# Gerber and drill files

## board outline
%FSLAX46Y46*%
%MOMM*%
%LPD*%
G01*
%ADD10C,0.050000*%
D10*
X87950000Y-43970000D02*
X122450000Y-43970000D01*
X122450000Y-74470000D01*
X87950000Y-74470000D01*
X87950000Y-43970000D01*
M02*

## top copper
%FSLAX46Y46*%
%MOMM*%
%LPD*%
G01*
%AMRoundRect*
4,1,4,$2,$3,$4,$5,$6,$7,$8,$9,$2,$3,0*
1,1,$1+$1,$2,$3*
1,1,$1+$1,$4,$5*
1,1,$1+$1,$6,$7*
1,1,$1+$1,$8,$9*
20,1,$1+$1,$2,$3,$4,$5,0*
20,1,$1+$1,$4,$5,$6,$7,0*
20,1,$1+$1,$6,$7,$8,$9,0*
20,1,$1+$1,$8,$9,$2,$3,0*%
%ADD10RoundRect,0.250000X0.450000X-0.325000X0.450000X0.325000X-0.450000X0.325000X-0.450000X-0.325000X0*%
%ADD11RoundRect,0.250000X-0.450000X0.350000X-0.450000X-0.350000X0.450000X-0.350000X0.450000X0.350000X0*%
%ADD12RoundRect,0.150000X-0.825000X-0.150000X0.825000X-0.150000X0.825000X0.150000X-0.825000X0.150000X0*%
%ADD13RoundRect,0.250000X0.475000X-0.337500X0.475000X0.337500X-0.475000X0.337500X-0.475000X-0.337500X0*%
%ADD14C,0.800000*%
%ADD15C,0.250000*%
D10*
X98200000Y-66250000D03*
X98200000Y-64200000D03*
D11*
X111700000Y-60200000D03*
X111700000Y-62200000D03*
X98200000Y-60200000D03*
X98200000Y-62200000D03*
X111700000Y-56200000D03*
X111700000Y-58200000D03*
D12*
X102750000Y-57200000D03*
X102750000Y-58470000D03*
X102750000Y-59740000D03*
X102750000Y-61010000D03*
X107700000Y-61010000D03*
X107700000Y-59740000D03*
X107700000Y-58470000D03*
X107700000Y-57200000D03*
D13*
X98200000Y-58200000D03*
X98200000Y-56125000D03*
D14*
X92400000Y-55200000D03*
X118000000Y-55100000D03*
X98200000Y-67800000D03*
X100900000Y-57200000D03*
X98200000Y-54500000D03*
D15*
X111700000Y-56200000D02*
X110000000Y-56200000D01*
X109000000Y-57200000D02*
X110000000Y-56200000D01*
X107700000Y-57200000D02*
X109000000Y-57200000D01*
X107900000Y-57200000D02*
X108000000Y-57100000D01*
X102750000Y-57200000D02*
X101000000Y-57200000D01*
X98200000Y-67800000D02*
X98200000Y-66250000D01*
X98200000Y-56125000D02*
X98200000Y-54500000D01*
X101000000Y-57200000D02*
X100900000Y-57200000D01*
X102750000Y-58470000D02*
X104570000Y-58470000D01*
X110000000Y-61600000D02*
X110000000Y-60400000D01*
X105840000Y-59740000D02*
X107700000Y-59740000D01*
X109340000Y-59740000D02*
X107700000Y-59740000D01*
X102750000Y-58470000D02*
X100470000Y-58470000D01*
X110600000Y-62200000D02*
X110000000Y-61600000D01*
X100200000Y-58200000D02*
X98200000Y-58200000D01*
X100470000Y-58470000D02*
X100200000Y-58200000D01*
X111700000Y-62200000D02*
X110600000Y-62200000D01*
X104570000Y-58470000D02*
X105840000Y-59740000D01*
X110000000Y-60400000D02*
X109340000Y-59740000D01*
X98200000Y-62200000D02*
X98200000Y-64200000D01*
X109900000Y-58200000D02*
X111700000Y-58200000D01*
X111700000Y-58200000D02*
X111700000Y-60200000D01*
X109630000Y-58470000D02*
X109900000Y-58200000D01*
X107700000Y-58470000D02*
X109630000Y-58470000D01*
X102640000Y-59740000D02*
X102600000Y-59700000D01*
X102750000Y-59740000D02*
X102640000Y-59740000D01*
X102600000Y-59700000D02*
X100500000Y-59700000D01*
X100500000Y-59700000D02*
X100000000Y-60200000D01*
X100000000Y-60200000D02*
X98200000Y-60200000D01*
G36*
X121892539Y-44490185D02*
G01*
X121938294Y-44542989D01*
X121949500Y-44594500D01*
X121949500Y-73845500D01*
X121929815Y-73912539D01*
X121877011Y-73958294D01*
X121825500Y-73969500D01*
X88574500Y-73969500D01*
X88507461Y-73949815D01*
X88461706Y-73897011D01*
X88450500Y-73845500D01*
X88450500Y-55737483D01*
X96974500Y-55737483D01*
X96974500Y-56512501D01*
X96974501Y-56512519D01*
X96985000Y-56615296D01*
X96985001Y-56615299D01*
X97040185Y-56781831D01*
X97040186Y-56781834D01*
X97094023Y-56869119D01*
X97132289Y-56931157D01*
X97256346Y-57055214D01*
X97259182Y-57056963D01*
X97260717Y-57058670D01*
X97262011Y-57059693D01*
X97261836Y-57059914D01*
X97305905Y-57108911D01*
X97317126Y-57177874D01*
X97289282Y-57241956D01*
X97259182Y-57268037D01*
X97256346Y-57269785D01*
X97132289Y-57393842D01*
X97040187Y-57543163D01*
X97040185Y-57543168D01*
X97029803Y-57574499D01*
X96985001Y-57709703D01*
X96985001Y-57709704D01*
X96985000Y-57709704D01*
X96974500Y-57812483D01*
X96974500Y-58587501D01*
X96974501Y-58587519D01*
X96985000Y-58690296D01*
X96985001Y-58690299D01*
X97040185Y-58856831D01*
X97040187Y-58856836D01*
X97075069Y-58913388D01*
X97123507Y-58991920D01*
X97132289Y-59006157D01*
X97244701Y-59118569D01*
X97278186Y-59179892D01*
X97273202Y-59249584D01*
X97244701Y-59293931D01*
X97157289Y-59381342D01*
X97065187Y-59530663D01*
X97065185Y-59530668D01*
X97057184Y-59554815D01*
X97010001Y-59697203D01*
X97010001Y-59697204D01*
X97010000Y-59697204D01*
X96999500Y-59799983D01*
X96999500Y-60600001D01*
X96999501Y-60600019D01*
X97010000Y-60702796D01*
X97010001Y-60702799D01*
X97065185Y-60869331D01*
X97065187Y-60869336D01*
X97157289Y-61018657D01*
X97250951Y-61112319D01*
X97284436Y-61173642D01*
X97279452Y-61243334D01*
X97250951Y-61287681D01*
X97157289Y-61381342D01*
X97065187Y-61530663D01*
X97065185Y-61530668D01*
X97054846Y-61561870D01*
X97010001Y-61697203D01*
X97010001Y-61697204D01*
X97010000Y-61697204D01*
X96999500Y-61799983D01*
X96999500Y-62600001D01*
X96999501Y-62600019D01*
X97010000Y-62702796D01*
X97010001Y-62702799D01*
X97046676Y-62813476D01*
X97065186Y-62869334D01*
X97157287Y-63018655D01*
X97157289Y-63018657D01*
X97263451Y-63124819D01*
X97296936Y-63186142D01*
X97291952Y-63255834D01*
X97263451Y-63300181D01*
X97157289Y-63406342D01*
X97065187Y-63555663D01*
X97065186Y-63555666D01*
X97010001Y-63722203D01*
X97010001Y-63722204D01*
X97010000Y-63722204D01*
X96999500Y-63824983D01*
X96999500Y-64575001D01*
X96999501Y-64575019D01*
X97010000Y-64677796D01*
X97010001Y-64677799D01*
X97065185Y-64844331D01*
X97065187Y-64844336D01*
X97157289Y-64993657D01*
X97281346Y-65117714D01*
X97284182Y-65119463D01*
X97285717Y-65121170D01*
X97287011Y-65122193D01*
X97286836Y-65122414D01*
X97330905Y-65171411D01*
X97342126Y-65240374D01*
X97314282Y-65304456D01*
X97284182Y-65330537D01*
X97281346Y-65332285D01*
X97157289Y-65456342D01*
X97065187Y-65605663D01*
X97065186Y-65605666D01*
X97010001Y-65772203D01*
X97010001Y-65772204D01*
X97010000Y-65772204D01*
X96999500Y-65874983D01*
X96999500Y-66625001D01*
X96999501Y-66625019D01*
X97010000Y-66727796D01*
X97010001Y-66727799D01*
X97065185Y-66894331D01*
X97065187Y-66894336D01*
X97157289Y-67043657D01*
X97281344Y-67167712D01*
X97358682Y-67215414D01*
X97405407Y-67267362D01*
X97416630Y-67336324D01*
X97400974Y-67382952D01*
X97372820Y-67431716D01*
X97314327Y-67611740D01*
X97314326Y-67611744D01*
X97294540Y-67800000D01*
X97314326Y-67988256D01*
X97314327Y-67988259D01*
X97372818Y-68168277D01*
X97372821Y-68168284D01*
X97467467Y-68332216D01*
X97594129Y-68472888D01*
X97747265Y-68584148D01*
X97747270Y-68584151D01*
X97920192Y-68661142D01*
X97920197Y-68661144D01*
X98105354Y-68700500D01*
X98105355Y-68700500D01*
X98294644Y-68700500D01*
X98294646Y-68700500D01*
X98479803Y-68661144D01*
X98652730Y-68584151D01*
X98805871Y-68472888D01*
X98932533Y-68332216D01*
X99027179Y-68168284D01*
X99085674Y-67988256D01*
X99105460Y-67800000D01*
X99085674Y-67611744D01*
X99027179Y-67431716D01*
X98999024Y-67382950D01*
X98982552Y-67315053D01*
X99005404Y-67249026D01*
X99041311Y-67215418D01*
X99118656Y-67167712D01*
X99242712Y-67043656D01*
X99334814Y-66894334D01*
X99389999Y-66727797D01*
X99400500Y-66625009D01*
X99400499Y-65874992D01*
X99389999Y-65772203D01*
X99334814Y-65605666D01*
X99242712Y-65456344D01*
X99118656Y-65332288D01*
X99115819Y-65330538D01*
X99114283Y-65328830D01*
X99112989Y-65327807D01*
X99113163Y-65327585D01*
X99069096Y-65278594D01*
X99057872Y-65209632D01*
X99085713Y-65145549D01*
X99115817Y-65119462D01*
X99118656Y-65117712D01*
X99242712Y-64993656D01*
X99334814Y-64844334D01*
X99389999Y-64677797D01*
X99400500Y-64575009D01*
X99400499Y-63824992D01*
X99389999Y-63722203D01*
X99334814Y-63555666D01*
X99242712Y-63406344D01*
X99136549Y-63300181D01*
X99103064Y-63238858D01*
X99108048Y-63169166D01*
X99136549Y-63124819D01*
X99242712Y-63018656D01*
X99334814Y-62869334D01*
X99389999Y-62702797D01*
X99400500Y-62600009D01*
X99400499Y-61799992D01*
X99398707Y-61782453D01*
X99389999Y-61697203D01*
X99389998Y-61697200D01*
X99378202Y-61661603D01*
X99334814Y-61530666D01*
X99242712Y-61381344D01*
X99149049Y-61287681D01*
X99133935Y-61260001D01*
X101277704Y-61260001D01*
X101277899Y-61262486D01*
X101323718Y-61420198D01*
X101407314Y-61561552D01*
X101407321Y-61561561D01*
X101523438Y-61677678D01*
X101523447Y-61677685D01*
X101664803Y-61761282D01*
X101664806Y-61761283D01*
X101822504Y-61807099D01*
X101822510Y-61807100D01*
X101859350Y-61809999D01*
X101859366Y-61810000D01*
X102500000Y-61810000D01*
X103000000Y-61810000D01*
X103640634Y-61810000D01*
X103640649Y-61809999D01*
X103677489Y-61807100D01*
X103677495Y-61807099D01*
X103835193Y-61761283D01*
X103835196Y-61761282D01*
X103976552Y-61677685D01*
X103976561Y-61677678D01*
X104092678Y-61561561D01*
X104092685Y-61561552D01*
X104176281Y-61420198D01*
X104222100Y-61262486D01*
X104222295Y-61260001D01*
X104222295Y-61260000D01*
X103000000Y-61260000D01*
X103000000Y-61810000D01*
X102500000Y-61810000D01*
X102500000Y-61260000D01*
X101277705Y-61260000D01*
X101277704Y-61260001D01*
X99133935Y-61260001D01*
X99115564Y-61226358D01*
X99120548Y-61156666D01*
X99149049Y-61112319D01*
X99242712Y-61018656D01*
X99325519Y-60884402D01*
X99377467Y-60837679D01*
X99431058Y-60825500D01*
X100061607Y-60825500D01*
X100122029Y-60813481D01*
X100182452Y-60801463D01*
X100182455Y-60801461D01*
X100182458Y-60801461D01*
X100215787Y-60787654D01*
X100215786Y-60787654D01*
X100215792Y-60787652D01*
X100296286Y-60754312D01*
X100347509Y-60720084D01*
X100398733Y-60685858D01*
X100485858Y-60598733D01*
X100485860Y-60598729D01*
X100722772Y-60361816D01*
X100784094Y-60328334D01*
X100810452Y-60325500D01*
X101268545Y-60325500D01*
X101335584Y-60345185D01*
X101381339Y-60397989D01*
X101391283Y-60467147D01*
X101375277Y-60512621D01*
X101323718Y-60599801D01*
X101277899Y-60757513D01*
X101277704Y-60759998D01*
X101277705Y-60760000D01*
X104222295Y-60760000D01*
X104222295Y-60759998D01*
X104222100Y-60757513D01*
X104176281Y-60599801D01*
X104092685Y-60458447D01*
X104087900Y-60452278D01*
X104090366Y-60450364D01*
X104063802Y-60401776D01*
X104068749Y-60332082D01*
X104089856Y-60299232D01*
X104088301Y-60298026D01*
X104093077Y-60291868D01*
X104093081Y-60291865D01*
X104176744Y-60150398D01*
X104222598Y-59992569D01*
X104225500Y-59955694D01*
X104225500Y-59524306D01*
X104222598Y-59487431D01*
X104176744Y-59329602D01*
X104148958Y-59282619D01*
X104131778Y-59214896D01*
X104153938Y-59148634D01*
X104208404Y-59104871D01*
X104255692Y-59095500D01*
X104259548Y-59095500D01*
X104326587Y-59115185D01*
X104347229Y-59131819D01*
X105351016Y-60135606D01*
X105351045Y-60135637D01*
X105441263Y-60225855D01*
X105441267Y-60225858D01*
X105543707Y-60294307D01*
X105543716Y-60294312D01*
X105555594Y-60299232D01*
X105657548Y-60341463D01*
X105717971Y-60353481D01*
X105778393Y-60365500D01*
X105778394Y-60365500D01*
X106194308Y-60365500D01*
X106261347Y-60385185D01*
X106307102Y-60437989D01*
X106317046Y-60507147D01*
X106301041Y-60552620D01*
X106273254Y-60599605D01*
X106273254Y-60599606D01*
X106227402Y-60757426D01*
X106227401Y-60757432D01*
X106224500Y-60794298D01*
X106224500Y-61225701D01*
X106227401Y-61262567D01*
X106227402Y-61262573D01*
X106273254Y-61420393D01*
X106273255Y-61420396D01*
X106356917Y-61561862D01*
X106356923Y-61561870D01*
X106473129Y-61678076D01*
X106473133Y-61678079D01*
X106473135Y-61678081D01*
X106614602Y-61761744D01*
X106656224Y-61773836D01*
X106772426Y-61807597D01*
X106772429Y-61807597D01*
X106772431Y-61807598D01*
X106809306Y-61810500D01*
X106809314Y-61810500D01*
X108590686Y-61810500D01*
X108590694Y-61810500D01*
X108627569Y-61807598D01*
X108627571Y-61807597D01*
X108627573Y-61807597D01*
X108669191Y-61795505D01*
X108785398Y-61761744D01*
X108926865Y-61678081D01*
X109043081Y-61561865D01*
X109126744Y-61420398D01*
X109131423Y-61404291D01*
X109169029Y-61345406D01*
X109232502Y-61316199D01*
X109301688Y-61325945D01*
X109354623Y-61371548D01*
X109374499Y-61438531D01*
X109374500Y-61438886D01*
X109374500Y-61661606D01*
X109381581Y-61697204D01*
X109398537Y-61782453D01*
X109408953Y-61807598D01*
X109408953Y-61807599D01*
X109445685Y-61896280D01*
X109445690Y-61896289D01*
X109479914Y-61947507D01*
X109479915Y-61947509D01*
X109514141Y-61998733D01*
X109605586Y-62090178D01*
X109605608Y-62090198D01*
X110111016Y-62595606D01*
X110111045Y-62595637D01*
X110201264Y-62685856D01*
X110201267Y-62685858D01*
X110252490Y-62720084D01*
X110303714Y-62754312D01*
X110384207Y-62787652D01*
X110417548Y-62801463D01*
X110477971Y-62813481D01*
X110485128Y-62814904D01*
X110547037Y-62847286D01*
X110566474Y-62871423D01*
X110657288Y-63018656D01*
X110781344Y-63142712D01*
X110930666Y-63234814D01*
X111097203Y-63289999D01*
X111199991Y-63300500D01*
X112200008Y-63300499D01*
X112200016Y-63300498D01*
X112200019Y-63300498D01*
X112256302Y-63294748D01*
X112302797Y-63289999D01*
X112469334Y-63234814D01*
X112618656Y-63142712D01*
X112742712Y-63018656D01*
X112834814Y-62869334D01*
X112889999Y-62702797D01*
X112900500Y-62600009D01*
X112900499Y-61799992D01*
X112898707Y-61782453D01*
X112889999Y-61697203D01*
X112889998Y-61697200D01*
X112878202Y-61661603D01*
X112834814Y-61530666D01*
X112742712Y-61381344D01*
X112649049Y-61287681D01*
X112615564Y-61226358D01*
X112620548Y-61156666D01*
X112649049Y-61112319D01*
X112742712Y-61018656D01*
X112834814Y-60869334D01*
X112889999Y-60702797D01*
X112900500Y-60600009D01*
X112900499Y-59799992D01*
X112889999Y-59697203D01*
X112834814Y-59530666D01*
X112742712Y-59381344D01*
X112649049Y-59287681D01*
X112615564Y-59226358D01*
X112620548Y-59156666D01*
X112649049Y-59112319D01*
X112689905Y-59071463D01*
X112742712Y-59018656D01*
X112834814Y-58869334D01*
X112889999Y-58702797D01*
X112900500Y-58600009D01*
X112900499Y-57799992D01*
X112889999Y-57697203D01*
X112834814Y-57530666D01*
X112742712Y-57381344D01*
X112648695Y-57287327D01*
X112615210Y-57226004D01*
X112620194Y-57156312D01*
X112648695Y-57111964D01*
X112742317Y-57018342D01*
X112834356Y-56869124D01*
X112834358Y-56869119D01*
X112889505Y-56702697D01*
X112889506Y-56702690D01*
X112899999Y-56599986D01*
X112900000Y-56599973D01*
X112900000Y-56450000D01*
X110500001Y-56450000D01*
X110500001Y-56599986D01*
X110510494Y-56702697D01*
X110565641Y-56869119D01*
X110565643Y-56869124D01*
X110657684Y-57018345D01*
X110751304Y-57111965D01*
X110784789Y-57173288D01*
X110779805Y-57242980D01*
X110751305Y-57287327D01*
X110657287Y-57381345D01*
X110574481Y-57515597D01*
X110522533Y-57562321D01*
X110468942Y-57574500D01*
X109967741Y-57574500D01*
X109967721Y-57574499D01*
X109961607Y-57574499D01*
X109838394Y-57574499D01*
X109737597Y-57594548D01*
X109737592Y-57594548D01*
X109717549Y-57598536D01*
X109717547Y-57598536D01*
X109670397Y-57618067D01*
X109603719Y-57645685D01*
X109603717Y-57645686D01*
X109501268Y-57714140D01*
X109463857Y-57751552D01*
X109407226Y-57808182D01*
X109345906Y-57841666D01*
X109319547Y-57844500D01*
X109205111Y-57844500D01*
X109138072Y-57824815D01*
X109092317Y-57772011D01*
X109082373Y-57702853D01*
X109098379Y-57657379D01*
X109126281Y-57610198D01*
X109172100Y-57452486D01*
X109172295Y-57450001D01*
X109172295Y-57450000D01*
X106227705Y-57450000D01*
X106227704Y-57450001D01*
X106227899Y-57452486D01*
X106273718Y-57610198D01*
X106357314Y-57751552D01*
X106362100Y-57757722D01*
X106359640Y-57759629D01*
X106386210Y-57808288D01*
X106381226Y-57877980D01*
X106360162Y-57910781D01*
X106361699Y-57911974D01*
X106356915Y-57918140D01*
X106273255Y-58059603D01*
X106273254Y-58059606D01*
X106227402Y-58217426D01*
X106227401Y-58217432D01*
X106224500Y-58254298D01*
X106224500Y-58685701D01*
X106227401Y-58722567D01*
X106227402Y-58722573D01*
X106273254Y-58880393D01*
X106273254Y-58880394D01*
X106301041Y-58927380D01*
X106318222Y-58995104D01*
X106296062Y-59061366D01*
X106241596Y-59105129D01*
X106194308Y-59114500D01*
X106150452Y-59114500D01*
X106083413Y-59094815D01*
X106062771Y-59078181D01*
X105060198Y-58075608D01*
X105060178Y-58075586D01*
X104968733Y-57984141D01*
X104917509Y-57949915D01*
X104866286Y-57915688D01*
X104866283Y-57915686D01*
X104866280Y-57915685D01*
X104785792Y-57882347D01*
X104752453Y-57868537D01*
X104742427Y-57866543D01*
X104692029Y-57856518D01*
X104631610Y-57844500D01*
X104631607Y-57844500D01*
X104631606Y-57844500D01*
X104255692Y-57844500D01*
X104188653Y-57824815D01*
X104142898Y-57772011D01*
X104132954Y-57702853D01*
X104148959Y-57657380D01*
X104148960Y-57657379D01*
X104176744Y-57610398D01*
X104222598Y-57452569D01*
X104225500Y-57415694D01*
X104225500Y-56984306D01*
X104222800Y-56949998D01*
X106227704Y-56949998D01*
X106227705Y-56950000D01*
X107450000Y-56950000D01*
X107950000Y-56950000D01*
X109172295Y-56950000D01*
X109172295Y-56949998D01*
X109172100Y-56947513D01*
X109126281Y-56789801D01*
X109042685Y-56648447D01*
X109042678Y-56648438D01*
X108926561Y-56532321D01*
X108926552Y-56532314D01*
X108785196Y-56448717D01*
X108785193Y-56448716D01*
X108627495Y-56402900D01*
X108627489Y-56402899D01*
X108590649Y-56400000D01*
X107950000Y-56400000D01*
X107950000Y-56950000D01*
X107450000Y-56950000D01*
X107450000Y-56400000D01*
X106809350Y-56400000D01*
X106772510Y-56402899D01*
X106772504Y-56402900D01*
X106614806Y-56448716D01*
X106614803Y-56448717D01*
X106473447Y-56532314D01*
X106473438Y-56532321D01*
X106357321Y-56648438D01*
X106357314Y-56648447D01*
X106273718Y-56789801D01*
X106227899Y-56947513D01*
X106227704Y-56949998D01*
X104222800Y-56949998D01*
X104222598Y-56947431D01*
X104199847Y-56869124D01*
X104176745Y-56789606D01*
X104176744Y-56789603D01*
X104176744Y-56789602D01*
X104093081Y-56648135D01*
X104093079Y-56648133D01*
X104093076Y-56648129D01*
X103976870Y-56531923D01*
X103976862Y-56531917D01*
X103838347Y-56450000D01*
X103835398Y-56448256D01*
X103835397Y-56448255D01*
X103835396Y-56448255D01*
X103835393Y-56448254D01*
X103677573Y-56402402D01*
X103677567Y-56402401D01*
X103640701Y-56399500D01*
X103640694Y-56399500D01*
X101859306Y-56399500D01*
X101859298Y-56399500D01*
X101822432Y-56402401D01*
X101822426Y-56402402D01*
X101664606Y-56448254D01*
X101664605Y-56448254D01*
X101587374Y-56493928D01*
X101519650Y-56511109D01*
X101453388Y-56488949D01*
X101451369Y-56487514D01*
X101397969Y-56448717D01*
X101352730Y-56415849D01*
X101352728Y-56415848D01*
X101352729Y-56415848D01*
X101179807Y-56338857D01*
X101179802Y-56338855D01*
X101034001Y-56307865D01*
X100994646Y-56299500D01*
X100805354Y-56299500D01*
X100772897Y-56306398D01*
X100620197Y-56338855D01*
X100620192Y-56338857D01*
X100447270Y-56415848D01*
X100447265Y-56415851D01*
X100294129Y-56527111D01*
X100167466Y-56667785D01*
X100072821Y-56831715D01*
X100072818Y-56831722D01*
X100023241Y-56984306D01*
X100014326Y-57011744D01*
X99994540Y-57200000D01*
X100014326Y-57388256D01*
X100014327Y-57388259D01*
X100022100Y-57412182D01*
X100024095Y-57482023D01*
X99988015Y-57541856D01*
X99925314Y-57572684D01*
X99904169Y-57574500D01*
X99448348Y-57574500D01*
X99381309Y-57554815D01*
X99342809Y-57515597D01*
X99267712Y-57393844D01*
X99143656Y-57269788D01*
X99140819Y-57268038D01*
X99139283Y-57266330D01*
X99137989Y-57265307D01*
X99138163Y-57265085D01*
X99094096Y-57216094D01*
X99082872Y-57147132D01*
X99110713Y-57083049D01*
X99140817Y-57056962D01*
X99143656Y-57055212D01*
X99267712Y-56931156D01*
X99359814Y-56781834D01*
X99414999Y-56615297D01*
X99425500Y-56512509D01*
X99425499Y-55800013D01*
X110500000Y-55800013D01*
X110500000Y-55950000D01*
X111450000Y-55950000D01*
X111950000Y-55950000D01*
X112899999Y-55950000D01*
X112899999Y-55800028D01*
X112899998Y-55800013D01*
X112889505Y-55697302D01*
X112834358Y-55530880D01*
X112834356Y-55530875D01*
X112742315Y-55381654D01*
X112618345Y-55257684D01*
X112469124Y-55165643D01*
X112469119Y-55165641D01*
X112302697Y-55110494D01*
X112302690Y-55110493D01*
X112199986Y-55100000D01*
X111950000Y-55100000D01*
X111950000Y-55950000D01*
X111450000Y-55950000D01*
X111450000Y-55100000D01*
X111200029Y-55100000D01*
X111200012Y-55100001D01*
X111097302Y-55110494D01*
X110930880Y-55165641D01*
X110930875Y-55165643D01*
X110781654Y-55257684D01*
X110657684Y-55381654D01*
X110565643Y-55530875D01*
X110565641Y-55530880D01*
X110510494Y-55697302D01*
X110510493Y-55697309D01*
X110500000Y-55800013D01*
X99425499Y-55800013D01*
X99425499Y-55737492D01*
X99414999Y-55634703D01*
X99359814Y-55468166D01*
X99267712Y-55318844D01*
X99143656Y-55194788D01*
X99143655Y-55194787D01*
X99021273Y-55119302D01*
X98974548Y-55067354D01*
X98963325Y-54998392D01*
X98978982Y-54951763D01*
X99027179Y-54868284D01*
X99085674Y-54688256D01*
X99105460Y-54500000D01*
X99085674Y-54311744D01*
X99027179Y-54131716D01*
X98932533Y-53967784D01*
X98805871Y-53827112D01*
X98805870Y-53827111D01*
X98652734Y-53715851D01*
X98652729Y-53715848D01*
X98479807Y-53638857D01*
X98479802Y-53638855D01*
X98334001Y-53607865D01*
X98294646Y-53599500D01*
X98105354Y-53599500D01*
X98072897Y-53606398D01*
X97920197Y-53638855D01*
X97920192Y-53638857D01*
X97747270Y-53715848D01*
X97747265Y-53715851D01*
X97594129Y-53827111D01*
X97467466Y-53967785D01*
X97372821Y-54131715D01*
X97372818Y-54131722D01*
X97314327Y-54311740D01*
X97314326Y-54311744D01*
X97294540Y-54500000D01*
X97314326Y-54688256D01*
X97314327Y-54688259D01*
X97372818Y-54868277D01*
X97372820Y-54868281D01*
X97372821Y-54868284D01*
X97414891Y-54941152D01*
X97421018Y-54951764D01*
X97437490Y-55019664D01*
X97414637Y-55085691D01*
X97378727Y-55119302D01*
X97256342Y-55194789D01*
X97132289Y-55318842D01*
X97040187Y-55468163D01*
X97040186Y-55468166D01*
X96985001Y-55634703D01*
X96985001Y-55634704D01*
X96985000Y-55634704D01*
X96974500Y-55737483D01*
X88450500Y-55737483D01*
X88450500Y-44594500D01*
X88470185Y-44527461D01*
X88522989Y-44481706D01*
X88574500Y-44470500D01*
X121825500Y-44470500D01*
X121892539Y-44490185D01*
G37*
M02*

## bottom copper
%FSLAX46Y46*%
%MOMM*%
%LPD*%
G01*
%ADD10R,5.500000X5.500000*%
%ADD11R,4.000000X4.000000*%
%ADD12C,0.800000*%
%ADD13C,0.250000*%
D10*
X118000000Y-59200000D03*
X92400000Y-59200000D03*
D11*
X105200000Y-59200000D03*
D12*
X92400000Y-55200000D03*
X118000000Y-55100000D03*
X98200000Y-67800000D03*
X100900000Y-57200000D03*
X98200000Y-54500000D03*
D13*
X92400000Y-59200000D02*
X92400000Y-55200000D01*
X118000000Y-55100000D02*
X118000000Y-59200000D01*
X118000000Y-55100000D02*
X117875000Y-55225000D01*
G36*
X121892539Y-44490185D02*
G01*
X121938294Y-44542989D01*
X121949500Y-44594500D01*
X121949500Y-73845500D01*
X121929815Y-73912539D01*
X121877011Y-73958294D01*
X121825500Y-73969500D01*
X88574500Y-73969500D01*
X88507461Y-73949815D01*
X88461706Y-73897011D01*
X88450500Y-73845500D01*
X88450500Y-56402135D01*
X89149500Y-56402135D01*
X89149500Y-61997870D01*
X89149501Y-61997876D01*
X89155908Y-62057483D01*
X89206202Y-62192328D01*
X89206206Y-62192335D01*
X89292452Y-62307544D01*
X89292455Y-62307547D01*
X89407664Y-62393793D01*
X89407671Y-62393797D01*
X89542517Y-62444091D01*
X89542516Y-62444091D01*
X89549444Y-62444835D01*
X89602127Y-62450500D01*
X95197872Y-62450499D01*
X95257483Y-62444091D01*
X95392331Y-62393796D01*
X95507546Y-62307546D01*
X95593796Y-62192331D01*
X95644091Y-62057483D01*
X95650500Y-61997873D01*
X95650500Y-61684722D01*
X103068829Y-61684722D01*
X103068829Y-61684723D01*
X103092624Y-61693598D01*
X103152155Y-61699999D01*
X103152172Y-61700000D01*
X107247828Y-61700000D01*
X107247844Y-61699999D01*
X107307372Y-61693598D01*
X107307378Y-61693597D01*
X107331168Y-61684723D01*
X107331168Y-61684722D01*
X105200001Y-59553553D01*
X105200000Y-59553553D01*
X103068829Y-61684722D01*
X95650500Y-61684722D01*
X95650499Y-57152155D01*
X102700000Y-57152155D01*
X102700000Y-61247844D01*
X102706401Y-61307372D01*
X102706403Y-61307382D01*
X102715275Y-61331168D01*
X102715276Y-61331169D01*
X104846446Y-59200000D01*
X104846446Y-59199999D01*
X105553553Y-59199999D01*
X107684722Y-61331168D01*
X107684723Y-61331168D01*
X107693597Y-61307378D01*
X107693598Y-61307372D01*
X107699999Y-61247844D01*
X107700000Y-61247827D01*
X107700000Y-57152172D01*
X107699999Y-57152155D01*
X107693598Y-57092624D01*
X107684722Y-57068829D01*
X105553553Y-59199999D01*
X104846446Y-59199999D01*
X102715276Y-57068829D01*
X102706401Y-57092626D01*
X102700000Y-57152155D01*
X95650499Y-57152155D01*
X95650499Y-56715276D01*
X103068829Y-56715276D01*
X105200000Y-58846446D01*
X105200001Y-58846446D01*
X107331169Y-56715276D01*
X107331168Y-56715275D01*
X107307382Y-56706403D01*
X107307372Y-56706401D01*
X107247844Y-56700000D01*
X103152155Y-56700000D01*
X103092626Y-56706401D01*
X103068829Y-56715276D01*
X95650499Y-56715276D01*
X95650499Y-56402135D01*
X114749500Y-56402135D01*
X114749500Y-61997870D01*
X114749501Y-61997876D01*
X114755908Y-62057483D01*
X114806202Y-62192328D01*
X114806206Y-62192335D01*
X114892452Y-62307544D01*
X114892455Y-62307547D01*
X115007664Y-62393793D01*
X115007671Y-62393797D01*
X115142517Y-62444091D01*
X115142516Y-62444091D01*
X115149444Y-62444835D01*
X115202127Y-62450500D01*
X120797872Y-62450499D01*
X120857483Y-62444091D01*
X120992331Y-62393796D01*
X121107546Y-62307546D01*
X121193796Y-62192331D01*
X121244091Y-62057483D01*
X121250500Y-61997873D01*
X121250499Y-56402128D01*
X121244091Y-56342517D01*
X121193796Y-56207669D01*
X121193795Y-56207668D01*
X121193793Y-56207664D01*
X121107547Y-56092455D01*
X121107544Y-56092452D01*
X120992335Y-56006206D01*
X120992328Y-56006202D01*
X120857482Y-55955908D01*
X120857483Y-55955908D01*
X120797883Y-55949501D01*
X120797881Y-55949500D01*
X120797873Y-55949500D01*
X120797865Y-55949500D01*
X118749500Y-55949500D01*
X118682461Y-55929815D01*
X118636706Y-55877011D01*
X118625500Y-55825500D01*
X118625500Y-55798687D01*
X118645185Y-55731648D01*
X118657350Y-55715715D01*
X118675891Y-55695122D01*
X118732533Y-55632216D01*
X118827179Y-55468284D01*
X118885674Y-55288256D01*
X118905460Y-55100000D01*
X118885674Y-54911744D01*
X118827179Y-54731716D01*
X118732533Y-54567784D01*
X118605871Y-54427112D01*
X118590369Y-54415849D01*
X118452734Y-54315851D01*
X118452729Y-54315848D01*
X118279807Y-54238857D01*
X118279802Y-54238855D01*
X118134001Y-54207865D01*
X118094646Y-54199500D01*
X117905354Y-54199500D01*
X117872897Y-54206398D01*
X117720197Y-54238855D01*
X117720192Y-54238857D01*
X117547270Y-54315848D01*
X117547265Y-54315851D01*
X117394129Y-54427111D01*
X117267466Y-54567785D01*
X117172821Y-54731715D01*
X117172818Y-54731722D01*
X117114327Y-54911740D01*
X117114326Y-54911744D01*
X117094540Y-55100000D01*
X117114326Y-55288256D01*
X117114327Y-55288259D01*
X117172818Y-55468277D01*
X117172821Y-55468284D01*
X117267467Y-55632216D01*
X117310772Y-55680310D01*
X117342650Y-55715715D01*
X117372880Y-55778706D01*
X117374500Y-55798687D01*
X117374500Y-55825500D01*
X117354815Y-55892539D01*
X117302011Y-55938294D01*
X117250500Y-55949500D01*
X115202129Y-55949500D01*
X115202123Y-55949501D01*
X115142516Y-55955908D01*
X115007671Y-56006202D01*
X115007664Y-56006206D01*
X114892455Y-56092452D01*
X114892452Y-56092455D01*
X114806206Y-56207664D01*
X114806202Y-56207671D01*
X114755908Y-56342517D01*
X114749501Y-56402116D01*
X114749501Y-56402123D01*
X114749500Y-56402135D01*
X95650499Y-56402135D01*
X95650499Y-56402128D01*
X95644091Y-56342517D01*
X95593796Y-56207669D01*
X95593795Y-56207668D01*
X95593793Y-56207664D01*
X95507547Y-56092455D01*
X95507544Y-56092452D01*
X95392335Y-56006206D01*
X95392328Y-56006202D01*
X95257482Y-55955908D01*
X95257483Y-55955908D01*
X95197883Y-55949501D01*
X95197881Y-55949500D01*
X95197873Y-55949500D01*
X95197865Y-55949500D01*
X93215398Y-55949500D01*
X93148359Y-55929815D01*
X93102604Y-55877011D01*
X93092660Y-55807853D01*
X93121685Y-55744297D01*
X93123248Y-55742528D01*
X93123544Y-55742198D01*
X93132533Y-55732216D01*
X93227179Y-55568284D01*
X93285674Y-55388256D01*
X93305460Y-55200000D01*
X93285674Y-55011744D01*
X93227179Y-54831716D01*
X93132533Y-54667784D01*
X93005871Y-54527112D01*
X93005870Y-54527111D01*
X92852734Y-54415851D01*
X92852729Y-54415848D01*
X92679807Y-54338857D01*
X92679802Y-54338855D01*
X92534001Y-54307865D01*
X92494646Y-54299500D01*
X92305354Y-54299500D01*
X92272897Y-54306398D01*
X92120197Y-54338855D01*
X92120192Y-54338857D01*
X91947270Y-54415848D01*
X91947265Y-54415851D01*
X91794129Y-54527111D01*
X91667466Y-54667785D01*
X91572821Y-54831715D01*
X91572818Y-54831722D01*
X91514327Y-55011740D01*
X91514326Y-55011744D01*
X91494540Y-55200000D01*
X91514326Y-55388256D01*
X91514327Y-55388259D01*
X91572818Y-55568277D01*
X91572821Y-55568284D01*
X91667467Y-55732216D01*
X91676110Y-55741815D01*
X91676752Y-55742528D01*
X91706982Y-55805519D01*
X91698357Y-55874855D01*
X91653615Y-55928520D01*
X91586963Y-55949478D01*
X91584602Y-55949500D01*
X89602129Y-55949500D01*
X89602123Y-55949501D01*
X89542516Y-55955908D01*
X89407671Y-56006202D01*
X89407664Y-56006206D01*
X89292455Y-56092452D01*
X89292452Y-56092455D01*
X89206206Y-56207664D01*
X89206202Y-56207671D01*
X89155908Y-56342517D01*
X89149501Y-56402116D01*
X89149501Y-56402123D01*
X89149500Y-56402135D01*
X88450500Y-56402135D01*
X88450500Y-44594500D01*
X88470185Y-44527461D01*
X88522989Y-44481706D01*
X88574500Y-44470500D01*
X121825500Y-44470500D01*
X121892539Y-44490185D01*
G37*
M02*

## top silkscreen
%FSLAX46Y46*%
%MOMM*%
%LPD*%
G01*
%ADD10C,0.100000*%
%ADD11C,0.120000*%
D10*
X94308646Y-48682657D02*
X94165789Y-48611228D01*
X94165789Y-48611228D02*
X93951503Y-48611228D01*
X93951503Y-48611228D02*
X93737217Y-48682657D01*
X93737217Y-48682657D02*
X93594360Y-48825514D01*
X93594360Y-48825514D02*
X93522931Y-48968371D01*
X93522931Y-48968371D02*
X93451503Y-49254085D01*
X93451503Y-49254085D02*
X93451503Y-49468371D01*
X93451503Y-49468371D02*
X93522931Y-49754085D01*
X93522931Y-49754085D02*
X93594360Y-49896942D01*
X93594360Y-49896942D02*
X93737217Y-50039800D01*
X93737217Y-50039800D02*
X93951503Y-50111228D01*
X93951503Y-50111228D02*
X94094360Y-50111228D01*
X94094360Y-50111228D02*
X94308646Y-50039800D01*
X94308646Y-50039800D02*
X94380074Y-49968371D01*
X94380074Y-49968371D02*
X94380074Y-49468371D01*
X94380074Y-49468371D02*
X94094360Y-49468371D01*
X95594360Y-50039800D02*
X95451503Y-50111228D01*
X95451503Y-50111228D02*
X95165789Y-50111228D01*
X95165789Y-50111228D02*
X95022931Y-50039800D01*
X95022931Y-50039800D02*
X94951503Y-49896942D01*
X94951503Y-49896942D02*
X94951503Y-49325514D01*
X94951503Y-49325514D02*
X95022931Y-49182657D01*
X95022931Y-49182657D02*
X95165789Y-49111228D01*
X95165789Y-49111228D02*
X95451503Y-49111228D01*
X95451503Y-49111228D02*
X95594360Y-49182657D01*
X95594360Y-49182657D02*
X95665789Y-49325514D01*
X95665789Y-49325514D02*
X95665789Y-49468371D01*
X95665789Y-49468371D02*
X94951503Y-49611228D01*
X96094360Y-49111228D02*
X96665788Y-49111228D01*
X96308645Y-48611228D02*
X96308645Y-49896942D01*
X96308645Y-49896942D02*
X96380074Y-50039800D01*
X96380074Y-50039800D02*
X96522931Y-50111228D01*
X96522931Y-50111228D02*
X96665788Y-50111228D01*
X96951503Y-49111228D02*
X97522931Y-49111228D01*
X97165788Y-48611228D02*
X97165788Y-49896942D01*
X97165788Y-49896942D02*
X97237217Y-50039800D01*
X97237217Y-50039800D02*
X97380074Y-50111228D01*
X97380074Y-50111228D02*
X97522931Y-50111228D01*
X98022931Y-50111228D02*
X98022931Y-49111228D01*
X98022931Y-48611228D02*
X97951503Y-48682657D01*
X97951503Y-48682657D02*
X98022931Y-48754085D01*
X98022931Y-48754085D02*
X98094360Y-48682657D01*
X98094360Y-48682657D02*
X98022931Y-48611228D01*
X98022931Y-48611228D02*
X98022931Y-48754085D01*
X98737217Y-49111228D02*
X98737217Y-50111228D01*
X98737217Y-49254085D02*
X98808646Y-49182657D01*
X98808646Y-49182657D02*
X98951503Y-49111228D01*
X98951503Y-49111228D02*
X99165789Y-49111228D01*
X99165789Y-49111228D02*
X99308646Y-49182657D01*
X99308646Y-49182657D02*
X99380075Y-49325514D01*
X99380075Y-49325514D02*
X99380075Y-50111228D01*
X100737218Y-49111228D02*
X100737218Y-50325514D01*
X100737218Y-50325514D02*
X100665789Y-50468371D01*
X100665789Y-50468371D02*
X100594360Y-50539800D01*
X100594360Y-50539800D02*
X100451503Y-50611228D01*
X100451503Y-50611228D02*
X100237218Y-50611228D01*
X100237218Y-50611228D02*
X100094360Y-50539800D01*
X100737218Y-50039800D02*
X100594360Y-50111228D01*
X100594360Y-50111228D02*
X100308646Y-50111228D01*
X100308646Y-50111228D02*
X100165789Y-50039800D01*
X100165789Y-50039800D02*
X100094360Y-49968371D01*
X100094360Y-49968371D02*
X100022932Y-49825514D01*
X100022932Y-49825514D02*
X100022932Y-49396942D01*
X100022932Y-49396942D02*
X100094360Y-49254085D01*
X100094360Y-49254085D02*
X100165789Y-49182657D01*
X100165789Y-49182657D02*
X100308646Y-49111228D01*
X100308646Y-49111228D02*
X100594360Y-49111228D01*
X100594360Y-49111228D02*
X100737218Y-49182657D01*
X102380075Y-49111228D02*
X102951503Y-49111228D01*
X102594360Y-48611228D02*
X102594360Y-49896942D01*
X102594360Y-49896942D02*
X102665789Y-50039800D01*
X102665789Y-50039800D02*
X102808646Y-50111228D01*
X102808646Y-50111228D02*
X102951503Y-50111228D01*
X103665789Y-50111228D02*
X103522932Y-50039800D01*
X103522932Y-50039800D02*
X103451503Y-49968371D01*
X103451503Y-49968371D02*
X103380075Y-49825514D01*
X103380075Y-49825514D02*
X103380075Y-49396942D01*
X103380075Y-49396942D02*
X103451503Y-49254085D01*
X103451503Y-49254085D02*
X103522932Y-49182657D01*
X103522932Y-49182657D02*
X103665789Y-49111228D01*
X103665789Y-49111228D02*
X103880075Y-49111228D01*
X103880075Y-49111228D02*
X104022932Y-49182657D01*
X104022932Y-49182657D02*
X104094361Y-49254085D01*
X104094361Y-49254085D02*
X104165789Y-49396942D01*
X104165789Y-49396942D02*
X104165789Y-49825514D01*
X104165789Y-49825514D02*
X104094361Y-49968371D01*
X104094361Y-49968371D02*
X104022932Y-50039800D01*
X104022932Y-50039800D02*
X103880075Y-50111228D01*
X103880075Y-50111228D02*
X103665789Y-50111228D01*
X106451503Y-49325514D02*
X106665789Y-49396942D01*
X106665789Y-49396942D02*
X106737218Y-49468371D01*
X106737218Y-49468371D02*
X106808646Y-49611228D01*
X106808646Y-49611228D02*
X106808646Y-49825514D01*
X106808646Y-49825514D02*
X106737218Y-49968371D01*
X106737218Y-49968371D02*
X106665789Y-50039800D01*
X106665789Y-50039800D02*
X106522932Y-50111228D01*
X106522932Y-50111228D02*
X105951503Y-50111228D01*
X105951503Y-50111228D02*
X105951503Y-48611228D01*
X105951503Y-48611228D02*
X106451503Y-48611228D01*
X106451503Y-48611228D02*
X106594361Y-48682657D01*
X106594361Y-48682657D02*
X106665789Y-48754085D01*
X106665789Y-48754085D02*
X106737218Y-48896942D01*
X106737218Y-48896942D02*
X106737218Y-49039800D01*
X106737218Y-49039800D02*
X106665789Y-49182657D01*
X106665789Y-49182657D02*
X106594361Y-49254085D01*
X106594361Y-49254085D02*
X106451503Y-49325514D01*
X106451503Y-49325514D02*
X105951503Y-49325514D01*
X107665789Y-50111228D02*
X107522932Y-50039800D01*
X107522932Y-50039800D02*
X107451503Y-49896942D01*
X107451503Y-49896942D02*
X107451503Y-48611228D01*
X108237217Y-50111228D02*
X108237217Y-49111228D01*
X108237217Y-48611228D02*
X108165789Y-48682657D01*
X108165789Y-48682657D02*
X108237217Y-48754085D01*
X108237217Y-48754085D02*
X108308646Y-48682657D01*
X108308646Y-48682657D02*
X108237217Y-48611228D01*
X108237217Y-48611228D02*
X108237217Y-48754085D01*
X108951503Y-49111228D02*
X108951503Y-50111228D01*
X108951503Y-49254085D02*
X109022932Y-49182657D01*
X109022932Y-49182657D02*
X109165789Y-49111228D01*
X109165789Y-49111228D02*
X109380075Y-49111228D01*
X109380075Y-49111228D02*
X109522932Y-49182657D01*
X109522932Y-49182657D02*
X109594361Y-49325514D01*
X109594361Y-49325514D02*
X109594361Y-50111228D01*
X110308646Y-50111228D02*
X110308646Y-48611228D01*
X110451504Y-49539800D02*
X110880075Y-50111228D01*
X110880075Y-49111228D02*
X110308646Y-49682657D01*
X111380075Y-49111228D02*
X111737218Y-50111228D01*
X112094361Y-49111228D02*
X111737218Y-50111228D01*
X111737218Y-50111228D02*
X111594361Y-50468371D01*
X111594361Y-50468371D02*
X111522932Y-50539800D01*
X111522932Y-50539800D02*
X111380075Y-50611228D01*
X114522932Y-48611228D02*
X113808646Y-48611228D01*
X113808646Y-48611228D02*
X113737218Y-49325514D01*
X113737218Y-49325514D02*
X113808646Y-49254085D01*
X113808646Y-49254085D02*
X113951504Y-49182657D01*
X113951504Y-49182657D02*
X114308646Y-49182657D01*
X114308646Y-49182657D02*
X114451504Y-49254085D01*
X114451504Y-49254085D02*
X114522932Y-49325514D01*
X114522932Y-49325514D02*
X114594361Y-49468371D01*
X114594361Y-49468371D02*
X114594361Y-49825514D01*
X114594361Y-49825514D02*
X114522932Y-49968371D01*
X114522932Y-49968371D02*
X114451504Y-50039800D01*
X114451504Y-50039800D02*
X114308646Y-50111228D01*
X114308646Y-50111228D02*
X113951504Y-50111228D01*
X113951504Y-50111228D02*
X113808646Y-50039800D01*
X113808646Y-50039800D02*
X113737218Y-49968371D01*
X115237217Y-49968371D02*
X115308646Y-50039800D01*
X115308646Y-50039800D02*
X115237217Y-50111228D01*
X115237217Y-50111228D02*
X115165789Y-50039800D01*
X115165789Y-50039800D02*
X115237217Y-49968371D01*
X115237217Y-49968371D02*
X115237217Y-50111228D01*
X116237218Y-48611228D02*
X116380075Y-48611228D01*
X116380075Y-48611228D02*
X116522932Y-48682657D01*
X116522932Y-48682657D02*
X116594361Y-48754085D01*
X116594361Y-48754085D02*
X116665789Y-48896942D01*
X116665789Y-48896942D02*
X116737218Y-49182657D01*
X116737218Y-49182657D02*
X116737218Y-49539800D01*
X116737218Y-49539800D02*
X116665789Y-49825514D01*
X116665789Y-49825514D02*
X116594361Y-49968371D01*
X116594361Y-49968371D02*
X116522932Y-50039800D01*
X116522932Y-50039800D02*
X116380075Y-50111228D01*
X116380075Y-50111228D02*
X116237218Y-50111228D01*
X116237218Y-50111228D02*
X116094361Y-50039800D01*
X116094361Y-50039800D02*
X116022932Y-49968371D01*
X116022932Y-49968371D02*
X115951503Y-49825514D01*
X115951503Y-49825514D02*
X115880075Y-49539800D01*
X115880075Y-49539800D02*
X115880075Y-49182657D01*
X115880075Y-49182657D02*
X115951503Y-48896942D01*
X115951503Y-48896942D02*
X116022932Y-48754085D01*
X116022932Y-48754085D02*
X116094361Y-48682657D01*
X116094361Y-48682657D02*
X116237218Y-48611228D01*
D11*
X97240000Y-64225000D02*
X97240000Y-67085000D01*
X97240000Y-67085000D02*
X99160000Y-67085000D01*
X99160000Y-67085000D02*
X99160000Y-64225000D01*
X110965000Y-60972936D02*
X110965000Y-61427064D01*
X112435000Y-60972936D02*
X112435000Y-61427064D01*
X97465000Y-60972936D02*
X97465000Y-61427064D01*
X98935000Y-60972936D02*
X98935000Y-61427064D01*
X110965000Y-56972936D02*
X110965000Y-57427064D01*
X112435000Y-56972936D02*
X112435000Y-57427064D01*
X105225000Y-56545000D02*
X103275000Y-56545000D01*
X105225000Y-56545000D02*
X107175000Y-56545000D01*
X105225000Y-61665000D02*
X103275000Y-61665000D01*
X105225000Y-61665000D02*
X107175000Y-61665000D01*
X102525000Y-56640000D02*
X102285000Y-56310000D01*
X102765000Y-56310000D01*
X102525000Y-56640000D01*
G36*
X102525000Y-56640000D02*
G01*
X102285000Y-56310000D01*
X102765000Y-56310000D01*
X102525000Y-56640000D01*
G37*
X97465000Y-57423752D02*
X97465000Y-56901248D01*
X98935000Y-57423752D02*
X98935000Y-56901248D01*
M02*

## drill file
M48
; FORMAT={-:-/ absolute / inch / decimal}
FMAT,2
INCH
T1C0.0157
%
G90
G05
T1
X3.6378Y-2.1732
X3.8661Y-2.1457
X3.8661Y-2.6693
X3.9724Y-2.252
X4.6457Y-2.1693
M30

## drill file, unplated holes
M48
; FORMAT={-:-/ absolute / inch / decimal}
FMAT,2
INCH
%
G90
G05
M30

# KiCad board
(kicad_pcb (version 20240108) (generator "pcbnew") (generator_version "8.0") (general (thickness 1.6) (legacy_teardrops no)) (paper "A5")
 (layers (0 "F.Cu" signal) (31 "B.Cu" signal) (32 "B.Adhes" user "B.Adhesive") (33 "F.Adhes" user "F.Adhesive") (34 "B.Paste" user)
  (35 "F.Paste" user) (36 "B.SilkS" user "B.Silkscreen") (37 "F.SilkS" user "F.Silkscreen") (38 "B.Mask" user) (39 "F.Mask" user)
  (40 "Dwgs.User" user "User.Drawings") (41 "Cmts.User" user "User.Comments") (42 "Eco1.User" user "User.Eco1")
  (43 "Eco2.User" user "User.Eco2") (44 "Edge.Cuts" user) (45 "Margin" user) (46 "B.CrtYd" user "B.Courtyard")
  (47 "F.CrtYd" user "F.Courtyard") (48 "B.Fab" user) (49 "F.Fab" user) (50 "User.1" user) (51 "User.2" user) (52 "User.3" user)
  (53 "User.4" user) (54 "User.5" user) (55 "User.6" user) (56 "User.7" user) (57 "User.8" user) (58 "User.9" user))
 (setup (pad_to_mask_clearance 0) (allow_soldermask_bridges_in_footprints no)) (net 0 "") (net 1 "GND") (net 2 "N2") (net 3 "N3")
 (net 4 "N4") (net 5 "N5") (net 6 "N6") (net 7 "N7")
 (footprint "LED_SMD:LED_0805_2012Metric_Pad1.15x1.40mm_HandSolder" (layer "F.Cu") (at 98.2 65.225 90)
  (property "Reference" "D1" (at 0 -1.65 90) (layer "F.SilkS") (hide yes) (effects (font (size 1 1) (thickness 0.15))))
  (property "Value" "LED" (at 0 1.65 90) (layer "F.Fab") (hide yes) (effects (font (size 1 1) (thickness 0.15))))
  (fp_line (start 1 -0.96) (end -1.86 -0.96) (stroke (width 0.12) (type solid)) (layer "F.SilkS"))
  (fp_line (start -1.86 -0.96) (end -1.86 0.96) (stroke (width 0.12) (type solid)) (layer "F.SilkS"))
  (fp_line (start -1.86 0.96) (end 1 0.96) (stroke (width 0.12) (type solid)) (layer "F.SilkS"))
  (pad "1" smd roundrect (at -1.025 0 90) (size 1.15 1.4) (layers "F.Cu" "F.Paste" "F.Mask") (roundrect_rratio 0.217391) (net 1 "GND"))
  (pad "2" smd roundrect (at 1.025 0 90) (size 1.15 1.4) (layers "F.Cu" "F.Paste" "F.Mask") (roundrect_rratio 0.217391) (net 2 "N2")))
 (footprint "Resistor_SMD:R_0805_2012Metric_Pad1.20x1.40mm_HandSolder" (layer "F.Cu") (at 111.7 61.2 -90)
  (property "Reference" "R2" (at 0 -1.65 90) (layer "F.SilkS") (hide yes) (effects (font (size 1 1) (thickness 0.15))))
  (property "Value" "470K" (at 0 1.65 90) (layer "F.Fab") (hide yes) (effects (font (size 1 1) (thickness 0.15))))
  (fp_line (start -0.227064 0.735) (end 0.227064 0.735) (stroke (width 0.12) (type solid)) (layer "F.SilkS"))
  (fp_line (start -0.227064 -0.735) (end 0.227064 -0.735) (stroke (width 0.12) (type solid)) (layer "F.SilkS"))
  (pad "1" smd roundrect (at -1 0 270) (size 1.2 1.4) (layers "F.Cu" "F.Paste" "F.Mask") (roundrect_rratio 0.208333) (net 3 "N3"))
  (pad "2" smd roundrect (at 1 0 270) (size 1.2 1.4) (layers "F.Cu" "F.Paste" "F.Mask") (roundrect_rratio 0.208333) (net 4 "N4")))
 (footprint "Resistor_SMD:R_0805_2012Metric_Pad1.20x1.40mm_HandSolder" (layer "F.Cu") (at 98.2 61.2 -90)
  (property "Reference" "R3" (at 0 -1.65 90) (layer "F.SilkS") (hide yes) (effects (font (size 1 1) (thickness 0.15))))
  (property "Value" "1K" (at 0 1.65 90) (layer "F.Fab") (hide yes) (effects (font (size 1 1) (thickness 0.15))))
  (fp_line (start -0.227064 0.735) (end 0.227064 0.735) (stroke (width 0.12) (type solid)) (layer "F.SilkS"))
  (fp_line (start -0.227064 -0.735) (end 0.227064 -0.735) (stroke (width 0.12) (type solid)) (layer "F.SilkS"))
  (pad "1" smd roundrect (at -1 0 270) (size 1.2 1.4) (layers "F.Cu" "F.Paste" "F.Mask") (roundrect_rratio 0.208333) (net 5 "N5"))
  (pad "2" smd roundrect (at 1 0 270) (size 1.2 1.4) (layers "F.Cu" "F.Paste" "F.Mask") (roundrect_rratio 0.208333) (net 2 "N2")))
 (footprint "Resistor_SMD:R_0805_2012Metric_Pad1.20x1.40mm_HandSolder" (layer "F.Cu") (at 111.7 57.2 -90)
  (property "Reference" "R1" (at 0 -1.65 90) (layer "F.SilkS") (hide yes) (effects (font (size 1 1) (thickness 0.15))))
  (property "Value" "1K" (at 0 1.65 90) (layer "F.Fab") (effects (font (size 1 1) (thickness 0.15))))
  (fp_line (start -0.227064 0.735) (end 0.227064 0.735) (stroke (width 0.12) (type solid)) (layer "F.SilkS"))
  (fp_line (start -0.227064 -0.735) (end 0.227064 -0.735) (stroke (width 0.12) (type solid)) (layer "F.SilkS"))
  (pad "1" smd roundrect (at -1 0 270) (size 1.2 1.4) (layers "F.Cu" "F.Paste" "F.Mask") (roundrect_rratio 0.208333) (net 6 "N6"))
  (pad "2" smd roundrect (at 1 0 270) (size 1.2 1.4) (layers "F.Cu" "F.Paste" "F.Mask") (roundrect_rratio 0.208333) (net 3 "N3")))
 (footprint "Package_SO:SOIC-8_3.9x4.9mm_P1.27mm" (layer "F.Cu") (at 105.225 59.105)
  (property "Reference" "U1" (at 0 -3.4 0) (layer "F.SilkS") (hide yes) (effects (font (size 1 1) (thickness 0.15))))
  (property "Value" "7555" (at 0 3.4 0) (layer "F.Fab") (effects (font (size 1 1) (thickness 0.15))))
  (fp_line (start 0 -2.56) (end -1.95 -2.56) (stroke (width 0.12) (type solid)) (layer "F.SilkS"))
  (fp_line (start 0 -2.56) (end 1.95 -2.56) (stroke (width 0.12) (type solid)) (layer "F.SilkS"))
  (fp_line (start 0 2.56) (end -1.95 2.56) (stroke (width 0.12) (type solid)) (layer "F.SilkS"))
  (fp_line (start 0 2.56) (end 1.95 2.56) (stroke (width 0.12) (type solid)) (layer "F.SilkS"))
  (fp_poly
   (pts (xy -2.7 -2.465) (xy -2.94 -2.795) (xy -2.46 -2.795) (xy -2.7 -2.465)) (stroke (width 0.12) (type solid)) (fill solid)
   (layer "F.SilkS"))
  (pad "1" smd roundrect (at -2.475 -1.905) (size 1.95 0.6) (layers "F.Cu" "F.Paste" "F.Mask") (roundrect_rratio 0.25) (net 1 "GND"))
  (pad "2" smd roundrect (at -2.475 -0.635) (size 1.95 0.6) (layers "F.Cu" "F.Paste" "F.Mask") (roundrect_rratio 0.25) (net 4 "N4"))
  (pad "3" smd roundrect (at -2.475 0.635) (size 1.95 0.6) (layers "F.Cu" "F.Paste" "F.Mask") (roundrect_rratio 0.25) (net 5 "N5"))
  (pad "4" smd roundrect (at -2.475 1.905) (size 1.95 0.6) (layers "F.Cu" "F.Paste" "F.Mask") (roundrect_rratio 0.25) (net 6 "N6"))
  (pad "5" smd roundrect (at 2.475 1.905) (size 1.95 0.6) (layers "F.Cu" "F.Paste" "F.Mask") (roundrect_rratio 0.25) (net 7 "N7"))
  (pad "6" smd roundrect (at 2.475 0.635) (size 1.95 0.6) (layers "F.Cu" "F.Paste" "F.Mask") (roundrect_rratio 0.25) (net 4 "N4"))
  (pad "7" smd roundrect (at 2.475 -0.635) (size 1.95 0.6) (layers "F.Cu" "F.Paste" "F.Mask") (roundrect_rratio 0.25) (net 3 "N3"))
  (pad "8" smd roundrect (at 2.475 -1.905) (size 1.95 0.6) (layers "F.Cu" "F.Paste" "F.Mask") (roundrect_rratio 0.25) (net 6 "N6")))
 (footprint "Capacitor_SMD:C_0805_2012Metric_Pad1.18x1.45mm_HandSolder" (layer "F.Cu") (at 98.2 57.1625 90)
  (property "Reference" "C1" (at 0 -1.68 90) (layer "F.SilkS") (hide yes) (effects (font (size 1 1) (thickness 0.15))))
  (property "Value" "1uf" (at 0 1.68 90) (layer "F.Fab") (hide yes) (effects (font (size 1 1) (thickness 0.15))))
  (fp_line (start -0.261252 -0.735) (end 0.261252 -0.735) (stroke (width 0.12) (type solid)) (layer "F.SilkS"))
  (fp_line (start -0.261252 0.735) (end 0.261252 0.735) (stroke (width 0.12) (type solid)) (layer "F.SilkS"))
  (pad "1" smd roundrect (at -1.0375 0 90) (size 1.175 1.45) (layers "F.Cu" "F.Paste" "F.Mask") (roundrect_rratio 0.212766) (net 4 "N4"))
  (pad "2" smd roundrect (at 1.0375 0 90) (size 1.175 1.45) (layers "F.Cu" "F.Paste" "F.Mask") (roundrect_rratio 0.212766) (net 1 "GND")))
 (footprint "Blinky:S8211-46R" (layer "B.Cu") (at 105.2 59.2 180)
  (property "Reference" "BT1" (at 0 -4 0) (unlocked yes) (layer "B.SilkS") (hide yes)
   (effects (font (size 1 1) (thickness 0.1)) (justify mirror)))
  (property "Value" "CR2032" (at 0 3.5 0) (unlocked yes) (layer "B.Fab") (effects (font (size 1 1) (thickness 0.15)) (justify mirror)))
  (pad "1" smd rect (at -12.8 0 180) (size 5.5 5.5) (layers "B.Cu" "B.Paste" "B.Mask") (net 6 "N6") (thermal_bridge_angle 45))
  (pad "1" smd rect (at 12.8 0 180) (size 5.5 5.5) (layers "B.Cu" "B.Paste" "B.Mask") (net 6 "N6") (thermal_bridge_angle 45))
  (pad "2" smd rect (at 0 0 180) (size 4 4) (layers "B.Cu" "B.Paste" "B.Mask") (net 1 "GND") (thermal_bridge_angle 45)))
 (gr_rect (start 87.95 43.97) (end 122.45 74.47) (stroke (width 0.05) (type default)) (fill none) (layer "Edge.Cuts"))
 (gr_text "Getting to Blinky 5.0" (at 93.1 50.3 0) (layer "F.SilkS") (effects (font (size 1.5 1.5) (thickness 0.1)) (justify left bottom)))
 (segment (start 111.7 56.2) (end 110 56.2) (width 0.25) (layer "F.Cu") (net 6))
 (segment (start 109 57.2) (end 110 56.2) (width 0.25) (layer "F.Cu") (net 6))
 (segment (start 107.7 57.2) (end 109 57.2) (width 0.25) (layer "F.Cu") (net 6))
 (segment (start 107.9 57.2) (end 108 57.1) (width 0.25) (layer "F.Cu") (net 6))
 (via (at 92.4 55.2) (size 0.8) (drill 0.4) (layers "F.Cu" "B.Cu") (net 6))
 (via (at 118 55.1) (size 0.8) (drill 0.4) (layers "F.Cu" "B.Cu") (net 6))
 (segment (start 92.4 59.2) (end 92.4 55.2) (width 0.25) (layer "B.Cu") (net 6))
 (segment (start 118 55.1) (end 118 59.2) (width 0.25) (layer "B.Cu") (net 6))
 (segment (start 118 55.1) (end 117.875 55.225) (width 0.25) (layer "B.Cu") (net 6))
 (segment (start 102.75 57.2) (end 101 57.2) (width 0.25) (layer "F.Cu") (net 1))
 (segment (start 98.2 67.8) (end 98.2 66.25) (width 0.25) (layer "F.Cu") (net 1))
 (segment (start 98.2 56.125) (end 98.2 54.5) (width 0.25) (layer "F.Cu") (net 1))
 (segment (start 101 57.2) (end 100.9 57.2) (width 0.25) (layer "F.Cu") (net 1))
 (via (at 98.2 67.8) (size 0.8) (drill 0.4) (layers "F.Cu" "B.Cu") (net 1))
 (via (at 100.9 57.2) (size 0.8) (drill 0.4) (layers "F.Cu" "B.Cu") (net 1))
 (via (at 98.2 54.5) (size 0.8) (drill 0.4) (layers "F.Cu" "B.Cu") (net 1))
 (segment (start 102.75 58.47) (end 104.57 58.47) (width 0.25) (layer "F.Cu") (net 4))
 (segment (start 110 61.6) (end 110 60.4) (width 0.25) (layer "F.Cu") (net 4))
 (segment (start 105.84 59.74) (end 107.7 59.74) (width 0.25) (layer "F.Cu") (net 4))
 (segment (start 109.34 59.74) (end 107.7 59.74) (width 0.25) (layer "F.Cu") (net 4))
 (segment (start 102.75 58.47) (end 100.47 58.47) (width 0.25) (layer "F.Cu") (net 4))
 (segment (start 110.6 62.2) (end 110 61.6) (width 0.25) (layer "F.Cu") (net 4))
 (segment (start 100.2 58.2) (end 98.2 58.2) (width 0.25) (layer "F.Cu") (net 4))
 (segment (start 100.47 58.47) (end 100.2 58.2) (width 0.25) (layer "F.Cu") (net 4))
 (segment (start 111.7 62.2) (end 110.6 62.2) (width 0.25) (layer "F.Cu") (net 4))
 (segment (start 104.57 58.47) (end 105.84 59.74) (width 0.25) (layer "F.Cu") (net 4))
 (segment (start 110 60.4) (end 109.34 59.74) (width 0.25) (layer "F.Cu") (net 4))
 (segment (start 98.2 62.2) (end 98.2 64.2) (width 0.25) (layer "F.Cu") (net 2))
 (segment (start 109.9 58.2) (end 111.7 58.2) (width 0.25) (layer "F.Cu") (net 3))
 (segment (start 111.7 58.2) (end 111.7 60.2) (width 0.25) (layer "F.Cu") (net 3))
 (segment (start 109.63 58.47) (end 109.9 58.2) (width 0.25) (layer "F.Cu") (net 3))
 (segment (start 107.7 58.47) (end 109.63 58.47) (width 0.25) (layer "F.Cu") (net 3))
 (segment (start 102.64 59.74) (end 102.6 59.7) (width 0.25) (layer "F.Cu") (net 5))
 (segment (start 102.75 59.74) (end 102.64 59.74) (width 0.25) (layer "F.Cu") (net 5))
 (segment (start 102.6 59.7) (end 100.5 59.7) (width 0.25) (layer "F.Cu") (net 5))
 (segment (start 100.5 59.7) (end 100 60.2) (width 0.25) (layer "F.Cu") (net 5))
 (segment (start 100 60.2) (end 98.2 60.2) (width 0.25) (layer "F.Cu") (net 5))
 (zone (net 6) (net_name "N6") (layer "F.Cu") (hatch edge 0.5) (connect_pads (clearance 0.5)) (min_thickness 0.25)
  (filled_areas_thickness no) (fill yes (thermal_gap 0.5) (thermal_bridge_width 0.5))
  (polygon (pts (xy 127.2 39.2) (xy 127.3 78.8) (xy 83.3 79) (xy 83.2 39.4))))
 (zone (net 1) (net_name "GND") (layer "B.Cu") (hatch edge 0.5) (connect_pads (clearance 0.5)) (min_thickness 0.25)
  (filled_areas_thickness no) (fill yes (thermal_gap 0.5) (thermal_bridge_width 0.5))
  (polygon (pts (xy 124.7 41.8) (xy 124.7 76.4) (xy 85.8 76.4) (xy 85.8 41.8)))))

